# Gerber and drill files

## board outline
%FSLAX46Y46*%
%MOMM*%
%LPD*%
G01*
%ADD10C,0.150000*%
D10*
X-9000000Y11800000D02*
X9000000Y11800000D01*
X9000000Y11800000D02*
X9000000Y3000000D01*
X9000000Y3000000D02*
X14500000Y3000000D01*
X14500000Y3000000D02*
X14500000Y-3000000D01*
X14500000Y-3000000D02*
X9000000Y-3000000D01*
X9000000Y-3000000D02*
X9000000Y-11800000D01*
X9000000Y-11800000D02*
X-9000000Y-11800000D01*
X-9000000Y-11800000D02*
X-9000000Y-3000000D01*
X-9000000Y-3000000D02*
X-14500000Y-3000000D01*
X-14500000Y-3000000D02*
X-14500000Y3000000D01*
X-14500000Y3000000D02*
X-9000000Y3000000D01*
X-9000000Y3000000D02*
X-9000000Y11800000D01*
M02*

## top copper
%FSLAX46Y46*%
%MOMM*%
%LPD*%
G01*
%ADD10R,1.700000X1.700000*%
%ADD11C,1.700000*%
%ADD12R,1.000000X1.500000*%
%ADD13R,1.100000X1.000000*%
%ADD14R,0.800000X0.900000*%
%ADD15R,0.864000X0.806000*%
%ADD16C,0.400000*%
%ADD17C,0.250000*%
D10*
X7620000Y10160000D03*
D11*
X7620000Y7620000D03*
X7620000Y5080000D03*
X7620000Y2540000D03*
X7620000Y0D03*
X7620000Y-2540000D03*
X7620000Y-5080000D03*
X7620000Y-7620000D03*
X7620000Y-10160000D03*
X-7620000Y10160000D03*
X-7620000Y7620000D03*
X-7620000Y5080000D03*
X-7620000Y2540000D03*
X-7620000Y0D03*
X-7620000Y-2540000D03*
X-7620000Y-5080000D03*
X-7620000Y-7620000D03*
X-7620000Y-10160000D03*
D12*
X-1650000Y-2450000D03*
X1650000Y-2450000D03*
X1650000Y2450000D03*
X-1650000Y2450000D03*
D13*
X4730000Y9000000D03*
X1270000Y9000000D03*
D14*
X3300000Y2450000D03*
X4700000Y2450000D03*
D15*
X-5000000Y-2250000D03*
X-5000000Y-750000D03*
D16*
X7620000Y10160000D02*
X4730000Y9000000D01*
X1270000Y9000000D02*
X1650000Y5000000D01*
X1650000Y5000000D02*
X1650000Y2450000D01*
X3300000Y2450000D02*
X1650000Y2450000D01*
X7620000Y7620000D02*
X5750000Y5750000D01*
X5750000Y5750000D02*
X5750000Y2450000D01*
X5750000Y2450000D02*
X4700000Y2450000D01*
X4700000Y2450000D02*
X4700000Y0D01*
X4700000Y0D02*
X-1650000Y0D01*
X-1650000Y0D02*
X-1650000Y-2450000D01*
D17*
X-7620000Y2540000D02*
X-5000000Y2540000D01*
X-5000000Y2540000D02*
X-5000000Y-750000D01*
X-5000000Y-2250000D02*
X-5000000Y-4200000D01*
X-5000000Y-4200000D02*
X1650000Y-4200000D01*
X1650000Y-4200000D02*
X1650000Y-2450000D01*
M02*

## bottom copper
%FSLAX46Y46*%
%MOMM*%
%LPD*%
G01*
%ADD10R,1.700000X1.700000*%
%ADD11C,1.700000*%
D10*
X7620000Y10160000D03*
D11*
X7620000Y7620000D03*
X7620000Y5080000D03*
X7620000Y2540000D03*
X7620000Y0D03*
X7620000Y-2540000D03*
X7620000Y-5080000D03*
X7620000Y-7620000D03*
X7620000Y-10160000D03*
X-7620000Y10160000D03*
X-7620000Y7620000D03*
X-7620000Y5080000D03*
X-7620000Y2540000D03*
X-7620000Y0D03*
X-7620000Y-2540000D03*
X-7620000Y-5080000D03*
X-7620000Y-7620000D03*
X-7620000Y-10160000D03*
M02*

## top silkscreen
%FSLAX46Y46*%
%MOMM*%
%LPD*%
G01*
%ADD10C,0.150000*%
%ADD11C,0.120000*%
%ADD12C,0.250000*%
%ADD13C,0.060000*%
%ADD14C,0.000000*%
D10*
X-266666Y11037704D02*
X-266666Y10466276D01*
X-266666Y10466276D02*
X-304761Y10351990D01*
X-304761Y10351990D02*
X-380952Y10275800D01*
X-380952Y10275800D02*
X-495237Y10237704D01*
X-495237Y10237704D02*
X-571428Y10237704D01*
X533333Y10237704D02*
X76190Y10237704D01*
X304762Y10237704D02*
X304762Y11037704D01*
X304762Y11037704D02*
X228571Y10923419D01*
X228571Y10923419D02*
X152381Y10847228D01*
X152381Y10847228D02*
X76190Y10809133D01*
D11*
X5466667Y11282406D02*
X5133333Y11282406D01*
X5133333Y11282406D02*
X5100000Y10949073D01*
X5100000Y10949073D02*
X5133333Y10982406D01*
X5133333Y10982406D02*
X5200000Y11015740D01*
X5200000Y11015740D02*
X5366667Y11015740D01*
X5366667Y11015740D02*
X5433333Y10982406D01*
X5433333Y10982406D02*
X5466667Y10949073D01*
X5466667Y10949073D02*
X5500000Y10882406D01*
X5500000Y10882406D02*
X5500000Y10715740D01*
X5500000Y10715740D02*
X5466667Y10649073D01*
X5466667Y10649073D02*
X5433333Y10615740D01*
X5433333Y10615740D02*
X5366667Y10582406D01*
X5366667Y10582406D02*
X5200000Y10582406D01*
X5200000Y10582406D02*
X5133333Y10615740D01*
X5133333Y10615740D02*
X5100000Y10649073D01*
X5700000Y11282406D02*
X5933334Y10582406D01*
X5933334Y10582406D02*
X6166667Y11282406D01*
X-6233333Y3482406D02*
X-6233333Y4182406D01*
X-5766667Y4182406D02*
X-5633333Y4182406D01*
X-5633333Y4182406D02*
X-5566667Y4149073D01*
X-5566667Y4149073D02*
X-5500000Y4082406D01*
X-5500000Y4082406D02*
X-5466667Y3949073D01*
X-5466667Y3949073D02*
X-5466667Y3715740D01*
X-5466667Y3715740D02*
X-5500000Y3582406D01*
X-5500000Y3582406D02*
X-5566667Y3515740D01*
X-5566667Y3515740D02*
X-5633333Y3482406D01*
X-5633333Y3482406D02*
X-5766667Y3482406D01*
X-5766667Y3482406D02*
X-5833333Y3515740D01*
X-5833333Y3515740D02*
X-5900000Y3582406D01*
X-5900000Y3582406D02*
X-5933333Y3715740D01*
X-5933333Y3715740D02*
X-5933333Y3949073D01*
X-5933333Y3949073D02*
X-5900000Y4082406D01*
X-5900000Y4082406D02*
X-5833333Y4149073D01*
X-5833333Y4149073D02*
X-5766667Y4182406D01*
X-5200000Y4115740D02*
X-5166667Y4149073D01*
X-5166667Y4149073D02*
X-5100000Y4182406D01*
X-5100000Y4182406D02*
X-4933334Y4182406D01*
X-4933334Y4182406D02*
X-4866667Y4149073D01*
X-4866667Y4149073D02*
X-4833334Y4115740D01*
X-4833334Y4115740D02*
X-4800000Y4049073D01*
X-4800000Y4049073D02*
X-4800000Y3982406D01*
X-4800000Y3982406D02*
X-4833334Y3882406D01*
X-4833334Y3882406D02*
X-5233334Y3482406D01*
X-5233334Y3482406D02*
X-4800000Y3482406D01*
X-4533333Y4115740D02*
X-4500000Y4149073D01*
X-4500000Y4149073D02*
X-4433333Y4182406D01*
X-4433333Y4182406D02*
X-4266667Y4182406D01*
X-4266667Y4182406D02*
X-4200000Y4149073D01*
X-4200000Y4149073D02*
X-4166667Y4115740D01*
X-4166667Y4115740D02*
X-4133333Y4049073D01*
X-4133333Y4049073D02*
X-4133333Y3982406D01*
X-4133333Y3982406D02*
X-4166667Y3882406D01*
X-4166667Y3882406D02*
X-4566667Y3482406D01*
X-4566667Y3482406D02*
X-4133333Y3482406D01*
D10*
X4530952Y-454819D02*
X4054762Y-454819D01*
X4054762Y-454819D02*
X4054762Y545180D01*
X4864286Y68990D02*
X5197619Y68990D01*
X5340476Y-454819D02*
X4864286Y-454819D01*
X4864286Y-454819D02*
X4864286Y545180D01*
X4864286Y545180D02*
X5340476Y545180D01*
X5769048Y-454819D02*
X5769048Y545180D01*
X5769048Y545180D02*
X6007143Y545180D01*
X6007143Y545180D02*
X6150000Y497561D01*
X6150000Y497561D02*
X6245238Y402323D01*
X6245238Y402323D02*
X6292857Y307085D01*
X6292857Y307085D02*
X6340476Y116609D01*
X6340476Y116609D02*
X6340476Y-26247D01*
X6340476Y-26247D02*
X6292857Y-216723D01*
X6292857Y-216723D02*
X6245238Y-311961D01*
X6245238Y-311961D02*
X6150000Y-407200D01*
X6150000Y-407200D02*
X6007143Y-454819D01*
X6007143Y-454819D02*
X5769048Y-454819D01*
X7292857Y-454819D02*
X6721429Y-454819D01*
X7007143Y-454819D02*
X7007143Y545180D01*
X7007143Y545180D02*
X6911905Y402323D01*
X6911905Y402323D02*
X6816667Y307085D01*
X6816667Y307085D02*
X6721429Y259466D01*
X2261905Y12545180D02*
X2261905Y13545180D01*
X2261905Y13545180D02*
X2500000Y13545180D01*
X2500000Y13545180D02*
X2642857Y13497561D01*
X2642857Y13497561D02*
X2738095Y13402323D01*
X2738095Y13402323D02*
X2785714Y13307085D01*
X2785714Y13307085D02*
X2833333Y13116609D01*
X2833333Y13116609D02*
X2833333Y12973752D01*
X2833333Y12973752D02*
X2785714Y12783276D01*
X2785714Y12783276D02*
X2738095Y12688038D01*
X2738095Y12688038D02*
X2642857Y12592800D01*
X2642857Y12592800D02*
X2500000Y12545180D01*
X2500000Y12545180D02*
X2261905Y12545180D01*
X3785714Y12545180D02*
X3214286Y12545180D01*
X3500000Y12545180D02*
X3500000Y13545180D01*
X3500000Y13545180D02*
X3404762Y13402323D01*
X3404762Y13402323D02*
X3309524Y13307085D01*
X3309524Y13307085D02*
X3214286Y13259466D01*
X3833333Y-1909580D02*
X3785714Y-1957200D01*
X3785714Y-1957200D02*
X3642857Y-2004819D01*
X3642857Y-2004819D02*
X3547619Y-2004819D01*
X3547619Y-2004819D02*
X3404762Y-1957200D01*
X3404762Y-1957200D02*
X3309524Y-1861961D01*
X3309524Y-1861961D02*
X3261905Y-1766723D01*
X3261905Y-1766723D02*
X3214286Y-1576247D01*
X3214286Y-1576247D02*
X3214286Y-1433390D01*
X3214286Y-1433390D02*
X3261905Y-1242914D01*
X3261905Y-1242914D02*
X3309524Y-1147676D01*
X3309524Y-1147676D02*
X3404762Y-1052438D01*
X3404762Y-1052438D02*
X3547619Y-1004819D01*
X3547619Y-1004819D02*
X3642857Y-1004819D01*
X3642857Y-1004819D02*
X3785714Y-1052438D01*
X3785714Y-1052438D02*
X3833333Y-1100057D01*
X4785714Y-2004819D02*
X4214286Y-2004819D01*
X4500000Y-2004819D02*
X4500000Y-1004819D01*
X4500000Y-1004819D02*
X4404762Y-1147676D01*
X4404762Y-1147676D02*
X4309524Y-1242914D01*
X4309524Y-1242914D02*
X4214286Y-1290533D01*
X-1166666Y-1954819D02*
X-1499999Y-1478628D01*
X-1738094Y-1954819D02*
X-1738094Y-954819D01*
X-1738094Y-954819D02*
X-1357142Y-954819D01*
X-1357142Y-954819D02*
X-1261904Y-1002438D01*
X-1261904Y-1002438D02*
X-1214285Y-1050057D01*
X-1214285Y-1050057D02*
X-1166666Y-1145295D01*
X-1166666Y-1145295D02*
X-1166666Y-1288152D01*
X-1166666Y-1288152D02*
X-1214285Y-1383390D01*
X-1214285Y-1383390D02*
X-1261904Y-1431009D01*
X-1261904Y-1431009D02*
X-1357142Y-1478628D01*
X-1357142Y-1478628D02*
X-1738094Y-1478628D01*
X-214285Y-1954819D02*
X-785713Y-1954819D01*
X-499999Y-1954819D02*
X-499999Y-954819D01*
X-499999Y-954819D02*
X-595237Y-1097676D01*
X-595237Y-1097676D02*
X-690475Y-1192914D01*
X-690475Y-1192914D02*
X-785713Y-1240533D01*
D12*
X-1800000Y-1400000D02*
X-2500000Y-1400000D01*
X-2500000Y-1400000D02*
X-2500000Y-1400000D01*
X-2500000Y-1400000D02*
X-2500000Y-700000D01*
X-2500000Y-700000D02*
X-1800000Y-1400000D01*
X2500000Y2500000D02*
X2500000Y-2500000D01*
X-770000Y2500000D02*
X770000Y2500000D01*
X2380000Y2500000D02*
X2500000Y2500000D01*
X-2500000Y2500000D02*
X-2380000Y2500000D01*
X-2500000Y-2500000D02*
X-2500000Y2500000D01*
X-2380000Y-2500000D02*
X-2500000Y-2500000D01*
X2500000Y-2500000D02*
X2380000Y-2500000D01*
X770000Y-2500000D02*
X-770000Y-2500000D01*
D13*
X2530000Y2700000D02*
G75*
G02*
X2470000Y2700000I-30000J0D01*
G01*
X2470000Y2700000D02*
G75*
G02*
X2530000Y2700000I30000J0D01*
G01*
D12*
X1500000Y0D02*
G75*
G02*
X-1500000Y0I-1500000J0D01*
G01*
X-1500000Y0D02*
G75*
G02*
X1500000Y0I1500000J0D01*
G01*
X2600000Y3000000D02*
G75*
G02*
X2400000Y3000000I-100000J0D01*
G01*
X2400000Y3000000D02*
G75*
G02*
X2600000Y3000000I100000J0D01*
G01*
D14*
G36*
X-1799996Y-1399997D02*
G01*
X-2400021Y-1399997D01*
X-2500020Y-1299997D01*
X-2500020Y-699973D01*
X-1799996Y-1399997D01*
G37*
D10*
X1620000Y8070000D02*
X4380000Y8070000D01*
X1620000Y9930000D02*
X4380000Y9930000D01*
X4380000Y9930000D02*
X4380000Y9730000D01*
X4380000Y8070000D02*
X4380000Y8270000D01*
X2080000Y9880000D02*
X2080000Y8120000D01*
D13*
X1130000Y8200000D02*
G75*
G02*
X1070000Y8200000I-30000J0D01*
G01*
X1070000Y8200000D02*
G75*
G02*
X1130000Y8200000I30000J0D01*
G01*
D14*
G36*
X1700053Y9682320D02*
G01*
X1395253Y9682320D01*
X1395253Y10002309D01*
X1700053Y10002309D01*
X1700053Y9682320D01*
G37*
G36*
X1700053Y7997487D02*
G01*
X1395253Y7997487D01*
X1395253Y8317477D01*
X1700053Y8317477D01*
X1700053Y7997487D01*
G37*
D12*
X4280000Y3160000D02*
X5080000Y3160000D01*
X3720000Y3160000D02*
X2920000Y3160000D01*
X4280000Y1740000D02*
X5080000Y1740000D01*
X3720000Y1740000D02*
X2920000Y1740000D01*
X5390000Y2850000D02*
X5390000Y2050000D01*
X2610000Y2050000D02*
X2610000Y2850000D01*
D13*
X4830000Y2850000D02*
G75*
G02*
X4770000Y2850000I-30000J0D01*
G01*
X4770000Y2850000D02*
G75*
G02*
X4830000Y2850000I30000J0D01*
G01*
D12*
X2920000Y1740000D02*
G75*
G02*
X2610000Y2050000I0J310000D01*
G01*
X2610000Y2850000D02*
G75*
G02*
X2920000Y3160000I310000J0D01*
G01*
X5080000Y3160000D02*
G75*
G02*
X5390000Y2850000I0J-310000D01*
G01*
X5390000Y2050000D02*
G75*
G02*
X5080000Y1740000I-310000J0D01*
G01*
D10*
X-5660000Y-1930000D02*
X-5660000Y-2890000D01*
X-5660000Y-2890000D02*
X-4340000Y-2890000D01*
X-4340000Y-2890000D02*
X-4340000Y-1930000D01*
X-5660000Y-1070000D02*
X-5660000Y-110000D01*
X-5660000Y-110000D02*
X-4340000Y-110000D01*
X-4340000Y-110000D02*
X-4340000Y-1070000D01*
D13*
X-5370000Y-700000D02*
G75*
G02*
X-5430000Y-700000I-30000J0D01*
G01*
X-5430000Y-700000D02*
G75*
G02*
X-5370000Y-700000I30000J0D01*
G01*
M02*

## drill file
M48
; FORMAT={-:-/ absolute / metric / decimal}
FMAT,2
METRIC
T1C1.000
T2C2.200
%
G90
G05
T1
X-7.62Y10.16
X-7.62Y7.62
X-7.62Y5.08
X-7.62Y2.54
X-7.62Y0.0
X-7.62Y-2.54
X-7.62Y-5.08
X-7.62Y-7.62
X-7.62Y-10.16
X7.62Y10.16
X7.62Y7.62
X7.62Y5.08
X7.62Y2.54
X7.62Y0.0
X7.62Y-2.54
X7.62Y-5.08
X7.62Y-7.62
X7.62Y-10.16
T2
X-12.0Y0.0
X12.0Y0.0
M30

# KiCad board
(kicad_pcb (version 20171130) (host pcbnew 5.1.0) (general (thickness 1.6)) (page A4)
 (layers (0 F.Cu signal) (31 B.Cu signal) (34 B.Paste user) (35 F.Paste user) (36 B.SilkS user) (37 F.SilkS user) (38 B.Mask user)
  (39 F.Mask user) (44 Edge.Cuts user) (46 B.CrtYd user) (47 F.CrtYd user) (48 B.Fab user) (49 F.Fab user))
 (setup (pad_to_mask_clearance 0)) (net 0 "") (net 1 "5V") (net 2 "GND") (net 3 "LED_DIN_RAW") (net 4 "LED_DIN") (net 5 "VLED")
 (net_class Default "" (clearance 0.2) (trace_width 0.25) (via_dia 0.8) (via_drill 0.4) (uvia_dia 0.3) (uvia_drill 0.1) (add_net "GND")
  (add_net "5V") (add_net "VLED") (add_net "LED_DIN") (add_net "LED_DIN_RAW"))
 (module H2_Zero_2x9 (layer F.Cu) (at 0 0)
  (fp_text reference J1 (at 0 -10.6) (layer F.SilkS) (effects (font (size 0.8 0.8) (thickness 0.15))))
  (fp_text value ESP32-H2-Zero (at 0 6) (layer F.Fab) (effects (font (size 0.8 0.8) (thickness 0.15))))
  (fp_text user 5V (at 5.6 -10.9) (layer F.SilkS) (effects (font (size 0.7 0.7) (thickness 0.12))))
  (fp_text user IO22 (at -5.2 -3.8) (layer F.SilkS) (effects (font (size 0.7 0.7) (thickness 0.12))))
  (pad "5V" thru_hole rect (at 7.62 -10.16) (size 1.7 1.7) (drill 1.0) (layers *.Cu *.Mask) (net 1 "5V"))
  (pad "GND" thru_hole circle (at 7.62 -7.62) (size 1.7 1.7) (drill 1.0) (layers *.Cu *.Mask) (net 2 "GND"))
  (pad "3V3" thru_hole circle (at 7.62 -5.08) (size 1.7 1.7) (drill 1.0) (layers *.Cu *.Mask))
  (pad "IO0" thru_hole circle (at 7.62 -2.54) (size 1.7 1.7) (drill 1.0) (layers *.Cu *.Mask))
  (pad "IO1" thru_hole circle (at 7.62 0.0) (size 1.7 1.7) (drill 1.0) (layers *.Cu *.Mask))
  (pad "IO2" thru_hole circle (at 7.62 2.54) (size 1.7 1.7) (drill 1.0) (layers *.Cu *.Mask))
  (pad "IO3" thru_hole circle (at 7.62 5.08) (size 1.7 1.7) (drill 1.0) (layers *.Cu *.Mask))
  (pad "IO4" thru_hole circle (at 7.62 7.62) (size 1.7 1.7) (drill 1.0) (layers *.Cu *.Mask))
  (pad "IO5" thru_hole circle (at 7.62 10.16) (size 1.7 1.7) (drill 1.0) (layers *.Cu *.Mask))
  (pad "IO24" thru_hole circle (at -7.62 -10.16) (size 1.7 1.7) (drill 1.0) (layers *.Cu *.Mask))
  (pad "IO23" thru_hole circle (at -7.62 -7.62) (size 1.7 1.7) (drill 1.0) (layers *.Cu *.Mask))
  (pad "IO25" thru_hole circle (at -7.62 -5.08) (size 1.7 1.7) (drill 1.0) (layers *.Cu *.Mask))
  (pad "IO22" thru_hole circle (at -7.62 -2.54) (size 1.7 1.7) (drill 1.0) (layers *.Cu *.Mask) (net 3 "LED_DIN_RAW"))
  (pad "IO14" thru_hole circle (at -7.62 0.0) (size 1.7 1.7) (drill 1.0) (layers *.Cu *.Mask))
  (pad "IO13" thru_hole circle (at -7.62 2.54) (size 1.7 1.7) (drill 1.0) (layers *.Cu *.Mask))
  (pad "IO12" thru_hole circle (at -7.62 5.08) (size 1.7 1.7) (drill 1.0) (layers *.Cu *.Mask))
  (pad "IO11" thru_hole circle (at -7.62 7.62) (size 1.7 1.7) (drill 1.0) (layers *.Cu *.Mask))
  (pad "IO10" thru_hole circle (at -7.62 10.16) (size 1.7 1.7) (drill 1.0) (layers *.Cu *.Mask)))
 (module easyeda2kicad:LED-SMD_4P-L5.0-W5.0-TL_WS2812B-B (layer F.Cu) (at 0 0 270)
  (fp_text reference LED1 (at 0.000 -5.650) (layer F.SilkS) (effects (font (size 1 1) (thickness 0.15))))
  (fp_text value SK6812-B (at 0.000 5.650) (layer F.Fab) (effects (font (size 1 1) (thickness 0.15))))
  (fp_line (start 1.40 1.80) (end 1.40 2.50) (layer F.SilkS) (width 0.25))
  (fp_line (start 1.40 2.50) (end 1.40 2.50) (layer F.SilkS) (width 0.25))
  (fp_line (start 1.40 2.50) (end 0.70 2.50) (layer F.SilkS) (width 0.25))
  (fp_line (start 0.70 2.50) (end 1.40 1.80) (layer F.SilkS) (width 0.25))
  (fp_line (start -2.50 -2.50) (end 2.50 -2.50) (layer F.SilkS) (width 0.25))
  (fp_line (start -2.50 0.77) (end -2.50 -0.77) (layer F.SilkS) (width 0.25))
  (fp_line (start -2.50 -2.38) (end -2.50 -2.50) (layer F.SilkS) (width 0.25))
  (fp_line (start -2.50 2.50) (end -2.50 2.38) (layer F.SilkS) (width 0.25))
  (fp_line (start 2.50 2.50) (end -2.50 2.50) (layer F.SilkS) (width 0.25))
  (fp_line (start 2.50 2.38) (end 2.50 2.50) (layer F.SilkS) (width 0.25))
  (fp_line (start 2.50 -2.50) (end 2.50 -2.38) (layer F.SilkS) (width 0.25))
  (fp_line (start 2.50 -0.77) (end 2.50 0.77) (layer F.SilkS) (width 0.25))
  (pad 3 smd rect (at 2.45 1.65 450.0) (size 1.500 1.000) (layers F.Cu F.Paste F.Mask) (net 2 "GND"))
  (pad 4 smd rect (at 2.45 -1.65 450.0) (size 1.500 1.000) (layers F.Cu F.Paste F.Mask) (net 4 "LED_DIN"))
  (pad 1 smd rect (at -2.45 -1.65 450.0) (size 1.500 1.000) (layers F.Cu F.Paste F.Mask) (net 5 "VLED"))
  (pad 2 smd rect (at -2.45 1.65 450.0) (size 1.500 1.000) (layers F.Cu F.Paste F.Mask))
  (fp_circle (center -2.70 -2.50) (end -2.67 -2.50) (layer F.SilkS) (width 0.06))
  (fp_circle (center 0.00 0.00) (end 1.50 0.00) (layer F.SilkS) (width 0.25))
  (fp_circle (center -3.00 -2.50) (end -2.90 -2.50) (layer F.SilkS) (width 0.25))
  (fp_poly
   (pts (xy 1.399997 1.799996) (xy 1.399997 2.400021) (xy 1.299997 2.500020) (xy 0.699973 2.500020) (xy 1.399997 1.799996))
   (stroke (width 0) (type solid)) (fill solid) (layer "F.SilkS")))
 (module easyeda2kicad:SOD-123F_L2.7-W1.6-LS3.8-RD (layer F.Cu) (at 3 -9 0)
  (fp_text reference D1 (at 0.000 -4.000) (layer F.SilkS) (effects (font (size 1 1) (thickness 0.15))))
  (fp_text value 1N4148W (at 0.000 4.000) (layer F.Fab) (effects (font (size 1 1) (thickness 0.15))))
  (fp_line (start -1.38 0.93) (end 1.38 0.93) (layer F.SilkS) (width 0.15))
  (fp_line (start -1.38 -0.93) (end 1.38 -0.93) (layer F.SilkS) (width 0.15))
  (fp_line (start 1.38 -0.93) (end 1.38 -0.73) (layer F.SilkS) (width 0.15))
  (fp_line (start 1.38 0.93) (end 1.38 0.73) (layer F.SilkS) (width 0.15))
  (fp_line (start -0.92 -0.88) (end -0.92 0.88) (layer F.SilkS) (width 0.15))
  (pad 2 smd rect (at 1.73 0.00 0.0) (size 1.100 1.000) (layers F.Cu F.Paste F.Mask) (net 1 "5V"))
  (pad 1 smd rect (at -1.73 0.00 0.0) (size 1.100 1.000) (layers F.Cu F.Paste F.Mask) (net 5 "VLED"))
  (fp_circle (center -1.90 0.80) (end -1.87 0.80) (layer F.SilkS) (width 0.06))
  (fp_poly
   (pts (xy -1.299947 -1.002309) (xy -1.299947 -0.682320) (xy -1.604747 -0.682320) (xy -1.604747 -1.002309) (xy -1.299947 -1.002309))
   (stroke (width 0) (type solid)) (fill solid) (layer "F.SilkS"))
  (fp_poly
   (pts (xy -1.299947 1.002513) (xy -1.299947 0.682523) (xy -1.604747 0.682523) (xy -1.604747 1.002513) (xy -1.299947 1.002513))
   (stroke (width 0) (type solid)) (fill solid) (layer "F.SilkS")))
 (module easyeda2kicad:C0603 (layer F.Cu) (at 4 -2.45 180)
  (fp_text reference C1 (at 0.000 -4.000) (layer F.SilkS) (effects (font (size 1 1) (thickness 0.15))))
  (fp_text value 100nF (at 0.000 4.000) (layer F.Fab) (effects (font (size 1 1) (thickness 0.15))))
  (fp_line (start -0.28 0.71) (end -1.08 0.71) (layer F.SilkS) (width 0.25))
  (fp_line (start 0.28 0.71) (end 1.08 0.71) (layer F.SilkS) (width 0.25))
  (fp_line (start -0.28 -0.71) (end -1.08 -0.71) (layer F.SilkS) (width 0.25))
  (fp_line (start 0.28 -0.71) (end 1.08 -0.71) (layer F.SilkS) (width 0.25))
  (fp_line (start -1.39 0.40) (end -1.39 -0.40) (layer F.SilkS) (width 0.25))
  (fp_line (start 1.39 -0.40) (end 1.39 0.40) (layer F.SilkS) (width 0.25))
  (pad 2 smd rect (at 0.70 0.00 180.0) (size 0.800 0.900) (layers F.Cu F.Paste F.Mask) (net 5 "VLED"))
  (pad 1 smd rect (at -0.70 0.00 180.0) (size 0.800 0.900) (layers F.Cu F.Paste F.Mask) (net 2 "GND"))
  (fp_circle (center -0.80 0.40) (end -0.77 0.40) (layer F.SilkS) (width 0.06))
  (fp_arc (start 1.08 -0.40) (end 1.39 -0.40) (angle -90.00) (layer F.SilkS) (width 0.25))
  (fp_arc (start 1.08 0.40) (end 1.08 0.71) (angle -90.00) (layer F.SilkS) (width 0.25))
  (fp_arc (start -1.08 0.40) (end -1.39 0.40) (angle -90.00) (layer F.SilkS) (width 0.25))
  (fp_arc (start -1.08 -0.40) (end -1.08 -0.71) (angle -90.00) (layer F.SilkS) (width 0.25)))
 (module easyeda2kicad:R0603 (layer F.Cu) (at -5 1.5 270)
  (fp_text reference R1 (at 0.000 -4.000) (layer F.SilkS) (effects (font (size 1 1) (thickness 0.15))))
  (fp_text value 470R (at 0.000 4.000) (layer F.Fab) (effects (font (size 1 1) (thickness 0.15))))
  (fp_line (start 0.43 0.66) (end 1.39 0.66) (layer F.SilkS) (width 0.15))
  (fp_line (start 1.39 0.66) (end 1.39 -0.66) (layer F.SilkS) (width 0.15))
  (fp_line (start 1.39 -0.66) (end 0.43 -0.66) (layer F.SilkS) (width 0.15))
  (fp_line (start -0.43 0.66) (end -1.39 0.66) (layer F.SilkS) (width 0.15))
  (fp_line (start -1.39 0.66) (end -1.39 -0.66) (layer F.SilkS) (width 0.15))
  (fp_line (start -1.39 -0.66) (end -0.43 -0.66) (layer F.SilkS) (width 0.15))
  (pad 2 smd rect (at 0.75 0.00 270.0) (size 0.806 0.864) (layers F.Cu F.Paste F.Mask) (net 4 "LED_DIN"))
  (pad 1 smd rect (at -0.75 0.00 270.0) (size 0.806 0.864) (layers F.Cu F.Paste F.Mask) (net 3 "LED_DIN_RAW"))
  (fp_circle (center -0.80 0.40) (end -0.77 0.40) (layer F.SilkS) (width 0.06)))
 (segment (start 7.62 -10.16) (end 4.73 -9) (width 0.4) (layer F.Cu) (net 1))
 (segment (start 1.27 -9) (end 1.65 -5) (width 0.4) (layer F.Cu) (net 5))
 (segment (start 1.65 -5) (end 1.65 -2.45) (width 0.4) (layer F.Cu) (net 5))
 (segment (start 3.3 -2.45) (end 1.65 -2.45) (width 0.4) (layer F.Cu) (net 5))
 (segment (start 7.62 -7.62) (end 5.75 -5.75) (width 0.4) (layer F.Cu) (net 2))
 (segment (start 5.75 -5.75) (end 5.75 -2.45) (width 0.4) (layer F.Cu) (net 2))
 (segment (start 5.75 -2.45) (end 4.7 -2.45) (width 0.4) (layer F.Cu) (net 2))
 (segment (start 4.7 -2.45) (end 4.7 0) (width 0.4) (layer F.Cu) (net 2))
 (segment (start 4.7 0) (end -1.65 0) (width 0.4) (layer F.Cu) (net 2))
 (segment (start -1.65 0) (end -1.65 2.45) (width 0.4) (layer F.Cu) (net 2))
 (segment (start -7.62 -2.54) (end -5 -2.54) (width 0.25) (layer F.Cu) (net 3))
 (segment (start -5 -2.54) (end -5 0.75) (width 0.25) (layer F.Cu) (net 3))
 (segment (start -5 2.25) (end -5 4.2) (width 0.25) (layer F.Cu) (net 4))
 (segment (start -5 4.2) (end 1.65 4.2) (width 0.25) (layer F.Cu) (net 4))
 (segment (start 1.65 4.2) (end 1.65 2.45) (width 0.25) (layer F.Cu) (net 4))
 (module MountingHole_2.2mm (layer F.Cu) (at -12 0)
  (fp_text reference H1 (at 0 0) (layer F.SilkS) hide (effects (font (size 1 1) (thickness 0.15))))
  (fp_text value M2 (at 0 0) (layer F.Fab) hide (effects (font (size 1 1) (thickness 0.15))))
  (pad "" np_thru_hole circle (at 0 0) (size 2.2 2.2) (drill 2.2) (layers *.Cu *.Mask)))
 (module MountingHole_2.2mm (layer F.Cu) (at 12 0)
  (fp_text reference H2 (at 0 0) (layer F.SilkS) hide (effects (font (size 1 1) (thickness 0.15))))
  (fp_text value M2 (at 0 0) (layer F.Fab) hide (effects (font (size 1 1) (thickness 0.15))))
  (pad "" np_thru_hole circle (at 0 0) (size 2.2 2.2) (drill 2.2) (layers *.Cu *.Mask)))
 (gr_line (start -9.0 -11.8) (end 9.0 -11.8) (layer Edge.Cuts) (width 0.15))
 (gr_line (start 9.0 -11.8) (end 9.0 -3.0) (layer Edge.Cuts) (width 0.15))
 (gr_line (start 9.0 -3.0) (end 14.5 -3.0) (layer Edge.Cuts) (width 0.15))
 (gr_line (start 14.5 -3.0) (end 14.5 3.0) (layer Edge.Cuts) (width 0.15))
 (gr_line (start 14.5 3.0) (end 9.0 3.0) (layer Edge.Cuts) (width 0.15))
 (gr_line (start 9.0 3.0) (end 9.0 11.8) (layer Edge.Cuts) (width 0.15))
 (gr_line (start 9.0 11.8) (end -9.0 11.8) (layer Edge.Cuts) (width 0.15))
 (gr_line (start -9.0 11.8) (end -9.0 3.0) (layer Edge.Cuts) (width 0.15))
 (gr_line (start -9.0 3.0) (end -14.5 3.0) (layer Edge.Cuts) (width 0.15))
 (gr_line (start -14.5 3.0) (end -14.5 -3.0) (layer Edge.Cuts) (width 0.15))
 (gr_line (start -14.5 -3.0) (end -9.0 -3.0) (layer Edge.Cuts) (width 0.15))
 (gr_line (start -9.0 -3.0) (end -9.0 -11.8) (layer Edge.Cuts) (width 0.15)))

